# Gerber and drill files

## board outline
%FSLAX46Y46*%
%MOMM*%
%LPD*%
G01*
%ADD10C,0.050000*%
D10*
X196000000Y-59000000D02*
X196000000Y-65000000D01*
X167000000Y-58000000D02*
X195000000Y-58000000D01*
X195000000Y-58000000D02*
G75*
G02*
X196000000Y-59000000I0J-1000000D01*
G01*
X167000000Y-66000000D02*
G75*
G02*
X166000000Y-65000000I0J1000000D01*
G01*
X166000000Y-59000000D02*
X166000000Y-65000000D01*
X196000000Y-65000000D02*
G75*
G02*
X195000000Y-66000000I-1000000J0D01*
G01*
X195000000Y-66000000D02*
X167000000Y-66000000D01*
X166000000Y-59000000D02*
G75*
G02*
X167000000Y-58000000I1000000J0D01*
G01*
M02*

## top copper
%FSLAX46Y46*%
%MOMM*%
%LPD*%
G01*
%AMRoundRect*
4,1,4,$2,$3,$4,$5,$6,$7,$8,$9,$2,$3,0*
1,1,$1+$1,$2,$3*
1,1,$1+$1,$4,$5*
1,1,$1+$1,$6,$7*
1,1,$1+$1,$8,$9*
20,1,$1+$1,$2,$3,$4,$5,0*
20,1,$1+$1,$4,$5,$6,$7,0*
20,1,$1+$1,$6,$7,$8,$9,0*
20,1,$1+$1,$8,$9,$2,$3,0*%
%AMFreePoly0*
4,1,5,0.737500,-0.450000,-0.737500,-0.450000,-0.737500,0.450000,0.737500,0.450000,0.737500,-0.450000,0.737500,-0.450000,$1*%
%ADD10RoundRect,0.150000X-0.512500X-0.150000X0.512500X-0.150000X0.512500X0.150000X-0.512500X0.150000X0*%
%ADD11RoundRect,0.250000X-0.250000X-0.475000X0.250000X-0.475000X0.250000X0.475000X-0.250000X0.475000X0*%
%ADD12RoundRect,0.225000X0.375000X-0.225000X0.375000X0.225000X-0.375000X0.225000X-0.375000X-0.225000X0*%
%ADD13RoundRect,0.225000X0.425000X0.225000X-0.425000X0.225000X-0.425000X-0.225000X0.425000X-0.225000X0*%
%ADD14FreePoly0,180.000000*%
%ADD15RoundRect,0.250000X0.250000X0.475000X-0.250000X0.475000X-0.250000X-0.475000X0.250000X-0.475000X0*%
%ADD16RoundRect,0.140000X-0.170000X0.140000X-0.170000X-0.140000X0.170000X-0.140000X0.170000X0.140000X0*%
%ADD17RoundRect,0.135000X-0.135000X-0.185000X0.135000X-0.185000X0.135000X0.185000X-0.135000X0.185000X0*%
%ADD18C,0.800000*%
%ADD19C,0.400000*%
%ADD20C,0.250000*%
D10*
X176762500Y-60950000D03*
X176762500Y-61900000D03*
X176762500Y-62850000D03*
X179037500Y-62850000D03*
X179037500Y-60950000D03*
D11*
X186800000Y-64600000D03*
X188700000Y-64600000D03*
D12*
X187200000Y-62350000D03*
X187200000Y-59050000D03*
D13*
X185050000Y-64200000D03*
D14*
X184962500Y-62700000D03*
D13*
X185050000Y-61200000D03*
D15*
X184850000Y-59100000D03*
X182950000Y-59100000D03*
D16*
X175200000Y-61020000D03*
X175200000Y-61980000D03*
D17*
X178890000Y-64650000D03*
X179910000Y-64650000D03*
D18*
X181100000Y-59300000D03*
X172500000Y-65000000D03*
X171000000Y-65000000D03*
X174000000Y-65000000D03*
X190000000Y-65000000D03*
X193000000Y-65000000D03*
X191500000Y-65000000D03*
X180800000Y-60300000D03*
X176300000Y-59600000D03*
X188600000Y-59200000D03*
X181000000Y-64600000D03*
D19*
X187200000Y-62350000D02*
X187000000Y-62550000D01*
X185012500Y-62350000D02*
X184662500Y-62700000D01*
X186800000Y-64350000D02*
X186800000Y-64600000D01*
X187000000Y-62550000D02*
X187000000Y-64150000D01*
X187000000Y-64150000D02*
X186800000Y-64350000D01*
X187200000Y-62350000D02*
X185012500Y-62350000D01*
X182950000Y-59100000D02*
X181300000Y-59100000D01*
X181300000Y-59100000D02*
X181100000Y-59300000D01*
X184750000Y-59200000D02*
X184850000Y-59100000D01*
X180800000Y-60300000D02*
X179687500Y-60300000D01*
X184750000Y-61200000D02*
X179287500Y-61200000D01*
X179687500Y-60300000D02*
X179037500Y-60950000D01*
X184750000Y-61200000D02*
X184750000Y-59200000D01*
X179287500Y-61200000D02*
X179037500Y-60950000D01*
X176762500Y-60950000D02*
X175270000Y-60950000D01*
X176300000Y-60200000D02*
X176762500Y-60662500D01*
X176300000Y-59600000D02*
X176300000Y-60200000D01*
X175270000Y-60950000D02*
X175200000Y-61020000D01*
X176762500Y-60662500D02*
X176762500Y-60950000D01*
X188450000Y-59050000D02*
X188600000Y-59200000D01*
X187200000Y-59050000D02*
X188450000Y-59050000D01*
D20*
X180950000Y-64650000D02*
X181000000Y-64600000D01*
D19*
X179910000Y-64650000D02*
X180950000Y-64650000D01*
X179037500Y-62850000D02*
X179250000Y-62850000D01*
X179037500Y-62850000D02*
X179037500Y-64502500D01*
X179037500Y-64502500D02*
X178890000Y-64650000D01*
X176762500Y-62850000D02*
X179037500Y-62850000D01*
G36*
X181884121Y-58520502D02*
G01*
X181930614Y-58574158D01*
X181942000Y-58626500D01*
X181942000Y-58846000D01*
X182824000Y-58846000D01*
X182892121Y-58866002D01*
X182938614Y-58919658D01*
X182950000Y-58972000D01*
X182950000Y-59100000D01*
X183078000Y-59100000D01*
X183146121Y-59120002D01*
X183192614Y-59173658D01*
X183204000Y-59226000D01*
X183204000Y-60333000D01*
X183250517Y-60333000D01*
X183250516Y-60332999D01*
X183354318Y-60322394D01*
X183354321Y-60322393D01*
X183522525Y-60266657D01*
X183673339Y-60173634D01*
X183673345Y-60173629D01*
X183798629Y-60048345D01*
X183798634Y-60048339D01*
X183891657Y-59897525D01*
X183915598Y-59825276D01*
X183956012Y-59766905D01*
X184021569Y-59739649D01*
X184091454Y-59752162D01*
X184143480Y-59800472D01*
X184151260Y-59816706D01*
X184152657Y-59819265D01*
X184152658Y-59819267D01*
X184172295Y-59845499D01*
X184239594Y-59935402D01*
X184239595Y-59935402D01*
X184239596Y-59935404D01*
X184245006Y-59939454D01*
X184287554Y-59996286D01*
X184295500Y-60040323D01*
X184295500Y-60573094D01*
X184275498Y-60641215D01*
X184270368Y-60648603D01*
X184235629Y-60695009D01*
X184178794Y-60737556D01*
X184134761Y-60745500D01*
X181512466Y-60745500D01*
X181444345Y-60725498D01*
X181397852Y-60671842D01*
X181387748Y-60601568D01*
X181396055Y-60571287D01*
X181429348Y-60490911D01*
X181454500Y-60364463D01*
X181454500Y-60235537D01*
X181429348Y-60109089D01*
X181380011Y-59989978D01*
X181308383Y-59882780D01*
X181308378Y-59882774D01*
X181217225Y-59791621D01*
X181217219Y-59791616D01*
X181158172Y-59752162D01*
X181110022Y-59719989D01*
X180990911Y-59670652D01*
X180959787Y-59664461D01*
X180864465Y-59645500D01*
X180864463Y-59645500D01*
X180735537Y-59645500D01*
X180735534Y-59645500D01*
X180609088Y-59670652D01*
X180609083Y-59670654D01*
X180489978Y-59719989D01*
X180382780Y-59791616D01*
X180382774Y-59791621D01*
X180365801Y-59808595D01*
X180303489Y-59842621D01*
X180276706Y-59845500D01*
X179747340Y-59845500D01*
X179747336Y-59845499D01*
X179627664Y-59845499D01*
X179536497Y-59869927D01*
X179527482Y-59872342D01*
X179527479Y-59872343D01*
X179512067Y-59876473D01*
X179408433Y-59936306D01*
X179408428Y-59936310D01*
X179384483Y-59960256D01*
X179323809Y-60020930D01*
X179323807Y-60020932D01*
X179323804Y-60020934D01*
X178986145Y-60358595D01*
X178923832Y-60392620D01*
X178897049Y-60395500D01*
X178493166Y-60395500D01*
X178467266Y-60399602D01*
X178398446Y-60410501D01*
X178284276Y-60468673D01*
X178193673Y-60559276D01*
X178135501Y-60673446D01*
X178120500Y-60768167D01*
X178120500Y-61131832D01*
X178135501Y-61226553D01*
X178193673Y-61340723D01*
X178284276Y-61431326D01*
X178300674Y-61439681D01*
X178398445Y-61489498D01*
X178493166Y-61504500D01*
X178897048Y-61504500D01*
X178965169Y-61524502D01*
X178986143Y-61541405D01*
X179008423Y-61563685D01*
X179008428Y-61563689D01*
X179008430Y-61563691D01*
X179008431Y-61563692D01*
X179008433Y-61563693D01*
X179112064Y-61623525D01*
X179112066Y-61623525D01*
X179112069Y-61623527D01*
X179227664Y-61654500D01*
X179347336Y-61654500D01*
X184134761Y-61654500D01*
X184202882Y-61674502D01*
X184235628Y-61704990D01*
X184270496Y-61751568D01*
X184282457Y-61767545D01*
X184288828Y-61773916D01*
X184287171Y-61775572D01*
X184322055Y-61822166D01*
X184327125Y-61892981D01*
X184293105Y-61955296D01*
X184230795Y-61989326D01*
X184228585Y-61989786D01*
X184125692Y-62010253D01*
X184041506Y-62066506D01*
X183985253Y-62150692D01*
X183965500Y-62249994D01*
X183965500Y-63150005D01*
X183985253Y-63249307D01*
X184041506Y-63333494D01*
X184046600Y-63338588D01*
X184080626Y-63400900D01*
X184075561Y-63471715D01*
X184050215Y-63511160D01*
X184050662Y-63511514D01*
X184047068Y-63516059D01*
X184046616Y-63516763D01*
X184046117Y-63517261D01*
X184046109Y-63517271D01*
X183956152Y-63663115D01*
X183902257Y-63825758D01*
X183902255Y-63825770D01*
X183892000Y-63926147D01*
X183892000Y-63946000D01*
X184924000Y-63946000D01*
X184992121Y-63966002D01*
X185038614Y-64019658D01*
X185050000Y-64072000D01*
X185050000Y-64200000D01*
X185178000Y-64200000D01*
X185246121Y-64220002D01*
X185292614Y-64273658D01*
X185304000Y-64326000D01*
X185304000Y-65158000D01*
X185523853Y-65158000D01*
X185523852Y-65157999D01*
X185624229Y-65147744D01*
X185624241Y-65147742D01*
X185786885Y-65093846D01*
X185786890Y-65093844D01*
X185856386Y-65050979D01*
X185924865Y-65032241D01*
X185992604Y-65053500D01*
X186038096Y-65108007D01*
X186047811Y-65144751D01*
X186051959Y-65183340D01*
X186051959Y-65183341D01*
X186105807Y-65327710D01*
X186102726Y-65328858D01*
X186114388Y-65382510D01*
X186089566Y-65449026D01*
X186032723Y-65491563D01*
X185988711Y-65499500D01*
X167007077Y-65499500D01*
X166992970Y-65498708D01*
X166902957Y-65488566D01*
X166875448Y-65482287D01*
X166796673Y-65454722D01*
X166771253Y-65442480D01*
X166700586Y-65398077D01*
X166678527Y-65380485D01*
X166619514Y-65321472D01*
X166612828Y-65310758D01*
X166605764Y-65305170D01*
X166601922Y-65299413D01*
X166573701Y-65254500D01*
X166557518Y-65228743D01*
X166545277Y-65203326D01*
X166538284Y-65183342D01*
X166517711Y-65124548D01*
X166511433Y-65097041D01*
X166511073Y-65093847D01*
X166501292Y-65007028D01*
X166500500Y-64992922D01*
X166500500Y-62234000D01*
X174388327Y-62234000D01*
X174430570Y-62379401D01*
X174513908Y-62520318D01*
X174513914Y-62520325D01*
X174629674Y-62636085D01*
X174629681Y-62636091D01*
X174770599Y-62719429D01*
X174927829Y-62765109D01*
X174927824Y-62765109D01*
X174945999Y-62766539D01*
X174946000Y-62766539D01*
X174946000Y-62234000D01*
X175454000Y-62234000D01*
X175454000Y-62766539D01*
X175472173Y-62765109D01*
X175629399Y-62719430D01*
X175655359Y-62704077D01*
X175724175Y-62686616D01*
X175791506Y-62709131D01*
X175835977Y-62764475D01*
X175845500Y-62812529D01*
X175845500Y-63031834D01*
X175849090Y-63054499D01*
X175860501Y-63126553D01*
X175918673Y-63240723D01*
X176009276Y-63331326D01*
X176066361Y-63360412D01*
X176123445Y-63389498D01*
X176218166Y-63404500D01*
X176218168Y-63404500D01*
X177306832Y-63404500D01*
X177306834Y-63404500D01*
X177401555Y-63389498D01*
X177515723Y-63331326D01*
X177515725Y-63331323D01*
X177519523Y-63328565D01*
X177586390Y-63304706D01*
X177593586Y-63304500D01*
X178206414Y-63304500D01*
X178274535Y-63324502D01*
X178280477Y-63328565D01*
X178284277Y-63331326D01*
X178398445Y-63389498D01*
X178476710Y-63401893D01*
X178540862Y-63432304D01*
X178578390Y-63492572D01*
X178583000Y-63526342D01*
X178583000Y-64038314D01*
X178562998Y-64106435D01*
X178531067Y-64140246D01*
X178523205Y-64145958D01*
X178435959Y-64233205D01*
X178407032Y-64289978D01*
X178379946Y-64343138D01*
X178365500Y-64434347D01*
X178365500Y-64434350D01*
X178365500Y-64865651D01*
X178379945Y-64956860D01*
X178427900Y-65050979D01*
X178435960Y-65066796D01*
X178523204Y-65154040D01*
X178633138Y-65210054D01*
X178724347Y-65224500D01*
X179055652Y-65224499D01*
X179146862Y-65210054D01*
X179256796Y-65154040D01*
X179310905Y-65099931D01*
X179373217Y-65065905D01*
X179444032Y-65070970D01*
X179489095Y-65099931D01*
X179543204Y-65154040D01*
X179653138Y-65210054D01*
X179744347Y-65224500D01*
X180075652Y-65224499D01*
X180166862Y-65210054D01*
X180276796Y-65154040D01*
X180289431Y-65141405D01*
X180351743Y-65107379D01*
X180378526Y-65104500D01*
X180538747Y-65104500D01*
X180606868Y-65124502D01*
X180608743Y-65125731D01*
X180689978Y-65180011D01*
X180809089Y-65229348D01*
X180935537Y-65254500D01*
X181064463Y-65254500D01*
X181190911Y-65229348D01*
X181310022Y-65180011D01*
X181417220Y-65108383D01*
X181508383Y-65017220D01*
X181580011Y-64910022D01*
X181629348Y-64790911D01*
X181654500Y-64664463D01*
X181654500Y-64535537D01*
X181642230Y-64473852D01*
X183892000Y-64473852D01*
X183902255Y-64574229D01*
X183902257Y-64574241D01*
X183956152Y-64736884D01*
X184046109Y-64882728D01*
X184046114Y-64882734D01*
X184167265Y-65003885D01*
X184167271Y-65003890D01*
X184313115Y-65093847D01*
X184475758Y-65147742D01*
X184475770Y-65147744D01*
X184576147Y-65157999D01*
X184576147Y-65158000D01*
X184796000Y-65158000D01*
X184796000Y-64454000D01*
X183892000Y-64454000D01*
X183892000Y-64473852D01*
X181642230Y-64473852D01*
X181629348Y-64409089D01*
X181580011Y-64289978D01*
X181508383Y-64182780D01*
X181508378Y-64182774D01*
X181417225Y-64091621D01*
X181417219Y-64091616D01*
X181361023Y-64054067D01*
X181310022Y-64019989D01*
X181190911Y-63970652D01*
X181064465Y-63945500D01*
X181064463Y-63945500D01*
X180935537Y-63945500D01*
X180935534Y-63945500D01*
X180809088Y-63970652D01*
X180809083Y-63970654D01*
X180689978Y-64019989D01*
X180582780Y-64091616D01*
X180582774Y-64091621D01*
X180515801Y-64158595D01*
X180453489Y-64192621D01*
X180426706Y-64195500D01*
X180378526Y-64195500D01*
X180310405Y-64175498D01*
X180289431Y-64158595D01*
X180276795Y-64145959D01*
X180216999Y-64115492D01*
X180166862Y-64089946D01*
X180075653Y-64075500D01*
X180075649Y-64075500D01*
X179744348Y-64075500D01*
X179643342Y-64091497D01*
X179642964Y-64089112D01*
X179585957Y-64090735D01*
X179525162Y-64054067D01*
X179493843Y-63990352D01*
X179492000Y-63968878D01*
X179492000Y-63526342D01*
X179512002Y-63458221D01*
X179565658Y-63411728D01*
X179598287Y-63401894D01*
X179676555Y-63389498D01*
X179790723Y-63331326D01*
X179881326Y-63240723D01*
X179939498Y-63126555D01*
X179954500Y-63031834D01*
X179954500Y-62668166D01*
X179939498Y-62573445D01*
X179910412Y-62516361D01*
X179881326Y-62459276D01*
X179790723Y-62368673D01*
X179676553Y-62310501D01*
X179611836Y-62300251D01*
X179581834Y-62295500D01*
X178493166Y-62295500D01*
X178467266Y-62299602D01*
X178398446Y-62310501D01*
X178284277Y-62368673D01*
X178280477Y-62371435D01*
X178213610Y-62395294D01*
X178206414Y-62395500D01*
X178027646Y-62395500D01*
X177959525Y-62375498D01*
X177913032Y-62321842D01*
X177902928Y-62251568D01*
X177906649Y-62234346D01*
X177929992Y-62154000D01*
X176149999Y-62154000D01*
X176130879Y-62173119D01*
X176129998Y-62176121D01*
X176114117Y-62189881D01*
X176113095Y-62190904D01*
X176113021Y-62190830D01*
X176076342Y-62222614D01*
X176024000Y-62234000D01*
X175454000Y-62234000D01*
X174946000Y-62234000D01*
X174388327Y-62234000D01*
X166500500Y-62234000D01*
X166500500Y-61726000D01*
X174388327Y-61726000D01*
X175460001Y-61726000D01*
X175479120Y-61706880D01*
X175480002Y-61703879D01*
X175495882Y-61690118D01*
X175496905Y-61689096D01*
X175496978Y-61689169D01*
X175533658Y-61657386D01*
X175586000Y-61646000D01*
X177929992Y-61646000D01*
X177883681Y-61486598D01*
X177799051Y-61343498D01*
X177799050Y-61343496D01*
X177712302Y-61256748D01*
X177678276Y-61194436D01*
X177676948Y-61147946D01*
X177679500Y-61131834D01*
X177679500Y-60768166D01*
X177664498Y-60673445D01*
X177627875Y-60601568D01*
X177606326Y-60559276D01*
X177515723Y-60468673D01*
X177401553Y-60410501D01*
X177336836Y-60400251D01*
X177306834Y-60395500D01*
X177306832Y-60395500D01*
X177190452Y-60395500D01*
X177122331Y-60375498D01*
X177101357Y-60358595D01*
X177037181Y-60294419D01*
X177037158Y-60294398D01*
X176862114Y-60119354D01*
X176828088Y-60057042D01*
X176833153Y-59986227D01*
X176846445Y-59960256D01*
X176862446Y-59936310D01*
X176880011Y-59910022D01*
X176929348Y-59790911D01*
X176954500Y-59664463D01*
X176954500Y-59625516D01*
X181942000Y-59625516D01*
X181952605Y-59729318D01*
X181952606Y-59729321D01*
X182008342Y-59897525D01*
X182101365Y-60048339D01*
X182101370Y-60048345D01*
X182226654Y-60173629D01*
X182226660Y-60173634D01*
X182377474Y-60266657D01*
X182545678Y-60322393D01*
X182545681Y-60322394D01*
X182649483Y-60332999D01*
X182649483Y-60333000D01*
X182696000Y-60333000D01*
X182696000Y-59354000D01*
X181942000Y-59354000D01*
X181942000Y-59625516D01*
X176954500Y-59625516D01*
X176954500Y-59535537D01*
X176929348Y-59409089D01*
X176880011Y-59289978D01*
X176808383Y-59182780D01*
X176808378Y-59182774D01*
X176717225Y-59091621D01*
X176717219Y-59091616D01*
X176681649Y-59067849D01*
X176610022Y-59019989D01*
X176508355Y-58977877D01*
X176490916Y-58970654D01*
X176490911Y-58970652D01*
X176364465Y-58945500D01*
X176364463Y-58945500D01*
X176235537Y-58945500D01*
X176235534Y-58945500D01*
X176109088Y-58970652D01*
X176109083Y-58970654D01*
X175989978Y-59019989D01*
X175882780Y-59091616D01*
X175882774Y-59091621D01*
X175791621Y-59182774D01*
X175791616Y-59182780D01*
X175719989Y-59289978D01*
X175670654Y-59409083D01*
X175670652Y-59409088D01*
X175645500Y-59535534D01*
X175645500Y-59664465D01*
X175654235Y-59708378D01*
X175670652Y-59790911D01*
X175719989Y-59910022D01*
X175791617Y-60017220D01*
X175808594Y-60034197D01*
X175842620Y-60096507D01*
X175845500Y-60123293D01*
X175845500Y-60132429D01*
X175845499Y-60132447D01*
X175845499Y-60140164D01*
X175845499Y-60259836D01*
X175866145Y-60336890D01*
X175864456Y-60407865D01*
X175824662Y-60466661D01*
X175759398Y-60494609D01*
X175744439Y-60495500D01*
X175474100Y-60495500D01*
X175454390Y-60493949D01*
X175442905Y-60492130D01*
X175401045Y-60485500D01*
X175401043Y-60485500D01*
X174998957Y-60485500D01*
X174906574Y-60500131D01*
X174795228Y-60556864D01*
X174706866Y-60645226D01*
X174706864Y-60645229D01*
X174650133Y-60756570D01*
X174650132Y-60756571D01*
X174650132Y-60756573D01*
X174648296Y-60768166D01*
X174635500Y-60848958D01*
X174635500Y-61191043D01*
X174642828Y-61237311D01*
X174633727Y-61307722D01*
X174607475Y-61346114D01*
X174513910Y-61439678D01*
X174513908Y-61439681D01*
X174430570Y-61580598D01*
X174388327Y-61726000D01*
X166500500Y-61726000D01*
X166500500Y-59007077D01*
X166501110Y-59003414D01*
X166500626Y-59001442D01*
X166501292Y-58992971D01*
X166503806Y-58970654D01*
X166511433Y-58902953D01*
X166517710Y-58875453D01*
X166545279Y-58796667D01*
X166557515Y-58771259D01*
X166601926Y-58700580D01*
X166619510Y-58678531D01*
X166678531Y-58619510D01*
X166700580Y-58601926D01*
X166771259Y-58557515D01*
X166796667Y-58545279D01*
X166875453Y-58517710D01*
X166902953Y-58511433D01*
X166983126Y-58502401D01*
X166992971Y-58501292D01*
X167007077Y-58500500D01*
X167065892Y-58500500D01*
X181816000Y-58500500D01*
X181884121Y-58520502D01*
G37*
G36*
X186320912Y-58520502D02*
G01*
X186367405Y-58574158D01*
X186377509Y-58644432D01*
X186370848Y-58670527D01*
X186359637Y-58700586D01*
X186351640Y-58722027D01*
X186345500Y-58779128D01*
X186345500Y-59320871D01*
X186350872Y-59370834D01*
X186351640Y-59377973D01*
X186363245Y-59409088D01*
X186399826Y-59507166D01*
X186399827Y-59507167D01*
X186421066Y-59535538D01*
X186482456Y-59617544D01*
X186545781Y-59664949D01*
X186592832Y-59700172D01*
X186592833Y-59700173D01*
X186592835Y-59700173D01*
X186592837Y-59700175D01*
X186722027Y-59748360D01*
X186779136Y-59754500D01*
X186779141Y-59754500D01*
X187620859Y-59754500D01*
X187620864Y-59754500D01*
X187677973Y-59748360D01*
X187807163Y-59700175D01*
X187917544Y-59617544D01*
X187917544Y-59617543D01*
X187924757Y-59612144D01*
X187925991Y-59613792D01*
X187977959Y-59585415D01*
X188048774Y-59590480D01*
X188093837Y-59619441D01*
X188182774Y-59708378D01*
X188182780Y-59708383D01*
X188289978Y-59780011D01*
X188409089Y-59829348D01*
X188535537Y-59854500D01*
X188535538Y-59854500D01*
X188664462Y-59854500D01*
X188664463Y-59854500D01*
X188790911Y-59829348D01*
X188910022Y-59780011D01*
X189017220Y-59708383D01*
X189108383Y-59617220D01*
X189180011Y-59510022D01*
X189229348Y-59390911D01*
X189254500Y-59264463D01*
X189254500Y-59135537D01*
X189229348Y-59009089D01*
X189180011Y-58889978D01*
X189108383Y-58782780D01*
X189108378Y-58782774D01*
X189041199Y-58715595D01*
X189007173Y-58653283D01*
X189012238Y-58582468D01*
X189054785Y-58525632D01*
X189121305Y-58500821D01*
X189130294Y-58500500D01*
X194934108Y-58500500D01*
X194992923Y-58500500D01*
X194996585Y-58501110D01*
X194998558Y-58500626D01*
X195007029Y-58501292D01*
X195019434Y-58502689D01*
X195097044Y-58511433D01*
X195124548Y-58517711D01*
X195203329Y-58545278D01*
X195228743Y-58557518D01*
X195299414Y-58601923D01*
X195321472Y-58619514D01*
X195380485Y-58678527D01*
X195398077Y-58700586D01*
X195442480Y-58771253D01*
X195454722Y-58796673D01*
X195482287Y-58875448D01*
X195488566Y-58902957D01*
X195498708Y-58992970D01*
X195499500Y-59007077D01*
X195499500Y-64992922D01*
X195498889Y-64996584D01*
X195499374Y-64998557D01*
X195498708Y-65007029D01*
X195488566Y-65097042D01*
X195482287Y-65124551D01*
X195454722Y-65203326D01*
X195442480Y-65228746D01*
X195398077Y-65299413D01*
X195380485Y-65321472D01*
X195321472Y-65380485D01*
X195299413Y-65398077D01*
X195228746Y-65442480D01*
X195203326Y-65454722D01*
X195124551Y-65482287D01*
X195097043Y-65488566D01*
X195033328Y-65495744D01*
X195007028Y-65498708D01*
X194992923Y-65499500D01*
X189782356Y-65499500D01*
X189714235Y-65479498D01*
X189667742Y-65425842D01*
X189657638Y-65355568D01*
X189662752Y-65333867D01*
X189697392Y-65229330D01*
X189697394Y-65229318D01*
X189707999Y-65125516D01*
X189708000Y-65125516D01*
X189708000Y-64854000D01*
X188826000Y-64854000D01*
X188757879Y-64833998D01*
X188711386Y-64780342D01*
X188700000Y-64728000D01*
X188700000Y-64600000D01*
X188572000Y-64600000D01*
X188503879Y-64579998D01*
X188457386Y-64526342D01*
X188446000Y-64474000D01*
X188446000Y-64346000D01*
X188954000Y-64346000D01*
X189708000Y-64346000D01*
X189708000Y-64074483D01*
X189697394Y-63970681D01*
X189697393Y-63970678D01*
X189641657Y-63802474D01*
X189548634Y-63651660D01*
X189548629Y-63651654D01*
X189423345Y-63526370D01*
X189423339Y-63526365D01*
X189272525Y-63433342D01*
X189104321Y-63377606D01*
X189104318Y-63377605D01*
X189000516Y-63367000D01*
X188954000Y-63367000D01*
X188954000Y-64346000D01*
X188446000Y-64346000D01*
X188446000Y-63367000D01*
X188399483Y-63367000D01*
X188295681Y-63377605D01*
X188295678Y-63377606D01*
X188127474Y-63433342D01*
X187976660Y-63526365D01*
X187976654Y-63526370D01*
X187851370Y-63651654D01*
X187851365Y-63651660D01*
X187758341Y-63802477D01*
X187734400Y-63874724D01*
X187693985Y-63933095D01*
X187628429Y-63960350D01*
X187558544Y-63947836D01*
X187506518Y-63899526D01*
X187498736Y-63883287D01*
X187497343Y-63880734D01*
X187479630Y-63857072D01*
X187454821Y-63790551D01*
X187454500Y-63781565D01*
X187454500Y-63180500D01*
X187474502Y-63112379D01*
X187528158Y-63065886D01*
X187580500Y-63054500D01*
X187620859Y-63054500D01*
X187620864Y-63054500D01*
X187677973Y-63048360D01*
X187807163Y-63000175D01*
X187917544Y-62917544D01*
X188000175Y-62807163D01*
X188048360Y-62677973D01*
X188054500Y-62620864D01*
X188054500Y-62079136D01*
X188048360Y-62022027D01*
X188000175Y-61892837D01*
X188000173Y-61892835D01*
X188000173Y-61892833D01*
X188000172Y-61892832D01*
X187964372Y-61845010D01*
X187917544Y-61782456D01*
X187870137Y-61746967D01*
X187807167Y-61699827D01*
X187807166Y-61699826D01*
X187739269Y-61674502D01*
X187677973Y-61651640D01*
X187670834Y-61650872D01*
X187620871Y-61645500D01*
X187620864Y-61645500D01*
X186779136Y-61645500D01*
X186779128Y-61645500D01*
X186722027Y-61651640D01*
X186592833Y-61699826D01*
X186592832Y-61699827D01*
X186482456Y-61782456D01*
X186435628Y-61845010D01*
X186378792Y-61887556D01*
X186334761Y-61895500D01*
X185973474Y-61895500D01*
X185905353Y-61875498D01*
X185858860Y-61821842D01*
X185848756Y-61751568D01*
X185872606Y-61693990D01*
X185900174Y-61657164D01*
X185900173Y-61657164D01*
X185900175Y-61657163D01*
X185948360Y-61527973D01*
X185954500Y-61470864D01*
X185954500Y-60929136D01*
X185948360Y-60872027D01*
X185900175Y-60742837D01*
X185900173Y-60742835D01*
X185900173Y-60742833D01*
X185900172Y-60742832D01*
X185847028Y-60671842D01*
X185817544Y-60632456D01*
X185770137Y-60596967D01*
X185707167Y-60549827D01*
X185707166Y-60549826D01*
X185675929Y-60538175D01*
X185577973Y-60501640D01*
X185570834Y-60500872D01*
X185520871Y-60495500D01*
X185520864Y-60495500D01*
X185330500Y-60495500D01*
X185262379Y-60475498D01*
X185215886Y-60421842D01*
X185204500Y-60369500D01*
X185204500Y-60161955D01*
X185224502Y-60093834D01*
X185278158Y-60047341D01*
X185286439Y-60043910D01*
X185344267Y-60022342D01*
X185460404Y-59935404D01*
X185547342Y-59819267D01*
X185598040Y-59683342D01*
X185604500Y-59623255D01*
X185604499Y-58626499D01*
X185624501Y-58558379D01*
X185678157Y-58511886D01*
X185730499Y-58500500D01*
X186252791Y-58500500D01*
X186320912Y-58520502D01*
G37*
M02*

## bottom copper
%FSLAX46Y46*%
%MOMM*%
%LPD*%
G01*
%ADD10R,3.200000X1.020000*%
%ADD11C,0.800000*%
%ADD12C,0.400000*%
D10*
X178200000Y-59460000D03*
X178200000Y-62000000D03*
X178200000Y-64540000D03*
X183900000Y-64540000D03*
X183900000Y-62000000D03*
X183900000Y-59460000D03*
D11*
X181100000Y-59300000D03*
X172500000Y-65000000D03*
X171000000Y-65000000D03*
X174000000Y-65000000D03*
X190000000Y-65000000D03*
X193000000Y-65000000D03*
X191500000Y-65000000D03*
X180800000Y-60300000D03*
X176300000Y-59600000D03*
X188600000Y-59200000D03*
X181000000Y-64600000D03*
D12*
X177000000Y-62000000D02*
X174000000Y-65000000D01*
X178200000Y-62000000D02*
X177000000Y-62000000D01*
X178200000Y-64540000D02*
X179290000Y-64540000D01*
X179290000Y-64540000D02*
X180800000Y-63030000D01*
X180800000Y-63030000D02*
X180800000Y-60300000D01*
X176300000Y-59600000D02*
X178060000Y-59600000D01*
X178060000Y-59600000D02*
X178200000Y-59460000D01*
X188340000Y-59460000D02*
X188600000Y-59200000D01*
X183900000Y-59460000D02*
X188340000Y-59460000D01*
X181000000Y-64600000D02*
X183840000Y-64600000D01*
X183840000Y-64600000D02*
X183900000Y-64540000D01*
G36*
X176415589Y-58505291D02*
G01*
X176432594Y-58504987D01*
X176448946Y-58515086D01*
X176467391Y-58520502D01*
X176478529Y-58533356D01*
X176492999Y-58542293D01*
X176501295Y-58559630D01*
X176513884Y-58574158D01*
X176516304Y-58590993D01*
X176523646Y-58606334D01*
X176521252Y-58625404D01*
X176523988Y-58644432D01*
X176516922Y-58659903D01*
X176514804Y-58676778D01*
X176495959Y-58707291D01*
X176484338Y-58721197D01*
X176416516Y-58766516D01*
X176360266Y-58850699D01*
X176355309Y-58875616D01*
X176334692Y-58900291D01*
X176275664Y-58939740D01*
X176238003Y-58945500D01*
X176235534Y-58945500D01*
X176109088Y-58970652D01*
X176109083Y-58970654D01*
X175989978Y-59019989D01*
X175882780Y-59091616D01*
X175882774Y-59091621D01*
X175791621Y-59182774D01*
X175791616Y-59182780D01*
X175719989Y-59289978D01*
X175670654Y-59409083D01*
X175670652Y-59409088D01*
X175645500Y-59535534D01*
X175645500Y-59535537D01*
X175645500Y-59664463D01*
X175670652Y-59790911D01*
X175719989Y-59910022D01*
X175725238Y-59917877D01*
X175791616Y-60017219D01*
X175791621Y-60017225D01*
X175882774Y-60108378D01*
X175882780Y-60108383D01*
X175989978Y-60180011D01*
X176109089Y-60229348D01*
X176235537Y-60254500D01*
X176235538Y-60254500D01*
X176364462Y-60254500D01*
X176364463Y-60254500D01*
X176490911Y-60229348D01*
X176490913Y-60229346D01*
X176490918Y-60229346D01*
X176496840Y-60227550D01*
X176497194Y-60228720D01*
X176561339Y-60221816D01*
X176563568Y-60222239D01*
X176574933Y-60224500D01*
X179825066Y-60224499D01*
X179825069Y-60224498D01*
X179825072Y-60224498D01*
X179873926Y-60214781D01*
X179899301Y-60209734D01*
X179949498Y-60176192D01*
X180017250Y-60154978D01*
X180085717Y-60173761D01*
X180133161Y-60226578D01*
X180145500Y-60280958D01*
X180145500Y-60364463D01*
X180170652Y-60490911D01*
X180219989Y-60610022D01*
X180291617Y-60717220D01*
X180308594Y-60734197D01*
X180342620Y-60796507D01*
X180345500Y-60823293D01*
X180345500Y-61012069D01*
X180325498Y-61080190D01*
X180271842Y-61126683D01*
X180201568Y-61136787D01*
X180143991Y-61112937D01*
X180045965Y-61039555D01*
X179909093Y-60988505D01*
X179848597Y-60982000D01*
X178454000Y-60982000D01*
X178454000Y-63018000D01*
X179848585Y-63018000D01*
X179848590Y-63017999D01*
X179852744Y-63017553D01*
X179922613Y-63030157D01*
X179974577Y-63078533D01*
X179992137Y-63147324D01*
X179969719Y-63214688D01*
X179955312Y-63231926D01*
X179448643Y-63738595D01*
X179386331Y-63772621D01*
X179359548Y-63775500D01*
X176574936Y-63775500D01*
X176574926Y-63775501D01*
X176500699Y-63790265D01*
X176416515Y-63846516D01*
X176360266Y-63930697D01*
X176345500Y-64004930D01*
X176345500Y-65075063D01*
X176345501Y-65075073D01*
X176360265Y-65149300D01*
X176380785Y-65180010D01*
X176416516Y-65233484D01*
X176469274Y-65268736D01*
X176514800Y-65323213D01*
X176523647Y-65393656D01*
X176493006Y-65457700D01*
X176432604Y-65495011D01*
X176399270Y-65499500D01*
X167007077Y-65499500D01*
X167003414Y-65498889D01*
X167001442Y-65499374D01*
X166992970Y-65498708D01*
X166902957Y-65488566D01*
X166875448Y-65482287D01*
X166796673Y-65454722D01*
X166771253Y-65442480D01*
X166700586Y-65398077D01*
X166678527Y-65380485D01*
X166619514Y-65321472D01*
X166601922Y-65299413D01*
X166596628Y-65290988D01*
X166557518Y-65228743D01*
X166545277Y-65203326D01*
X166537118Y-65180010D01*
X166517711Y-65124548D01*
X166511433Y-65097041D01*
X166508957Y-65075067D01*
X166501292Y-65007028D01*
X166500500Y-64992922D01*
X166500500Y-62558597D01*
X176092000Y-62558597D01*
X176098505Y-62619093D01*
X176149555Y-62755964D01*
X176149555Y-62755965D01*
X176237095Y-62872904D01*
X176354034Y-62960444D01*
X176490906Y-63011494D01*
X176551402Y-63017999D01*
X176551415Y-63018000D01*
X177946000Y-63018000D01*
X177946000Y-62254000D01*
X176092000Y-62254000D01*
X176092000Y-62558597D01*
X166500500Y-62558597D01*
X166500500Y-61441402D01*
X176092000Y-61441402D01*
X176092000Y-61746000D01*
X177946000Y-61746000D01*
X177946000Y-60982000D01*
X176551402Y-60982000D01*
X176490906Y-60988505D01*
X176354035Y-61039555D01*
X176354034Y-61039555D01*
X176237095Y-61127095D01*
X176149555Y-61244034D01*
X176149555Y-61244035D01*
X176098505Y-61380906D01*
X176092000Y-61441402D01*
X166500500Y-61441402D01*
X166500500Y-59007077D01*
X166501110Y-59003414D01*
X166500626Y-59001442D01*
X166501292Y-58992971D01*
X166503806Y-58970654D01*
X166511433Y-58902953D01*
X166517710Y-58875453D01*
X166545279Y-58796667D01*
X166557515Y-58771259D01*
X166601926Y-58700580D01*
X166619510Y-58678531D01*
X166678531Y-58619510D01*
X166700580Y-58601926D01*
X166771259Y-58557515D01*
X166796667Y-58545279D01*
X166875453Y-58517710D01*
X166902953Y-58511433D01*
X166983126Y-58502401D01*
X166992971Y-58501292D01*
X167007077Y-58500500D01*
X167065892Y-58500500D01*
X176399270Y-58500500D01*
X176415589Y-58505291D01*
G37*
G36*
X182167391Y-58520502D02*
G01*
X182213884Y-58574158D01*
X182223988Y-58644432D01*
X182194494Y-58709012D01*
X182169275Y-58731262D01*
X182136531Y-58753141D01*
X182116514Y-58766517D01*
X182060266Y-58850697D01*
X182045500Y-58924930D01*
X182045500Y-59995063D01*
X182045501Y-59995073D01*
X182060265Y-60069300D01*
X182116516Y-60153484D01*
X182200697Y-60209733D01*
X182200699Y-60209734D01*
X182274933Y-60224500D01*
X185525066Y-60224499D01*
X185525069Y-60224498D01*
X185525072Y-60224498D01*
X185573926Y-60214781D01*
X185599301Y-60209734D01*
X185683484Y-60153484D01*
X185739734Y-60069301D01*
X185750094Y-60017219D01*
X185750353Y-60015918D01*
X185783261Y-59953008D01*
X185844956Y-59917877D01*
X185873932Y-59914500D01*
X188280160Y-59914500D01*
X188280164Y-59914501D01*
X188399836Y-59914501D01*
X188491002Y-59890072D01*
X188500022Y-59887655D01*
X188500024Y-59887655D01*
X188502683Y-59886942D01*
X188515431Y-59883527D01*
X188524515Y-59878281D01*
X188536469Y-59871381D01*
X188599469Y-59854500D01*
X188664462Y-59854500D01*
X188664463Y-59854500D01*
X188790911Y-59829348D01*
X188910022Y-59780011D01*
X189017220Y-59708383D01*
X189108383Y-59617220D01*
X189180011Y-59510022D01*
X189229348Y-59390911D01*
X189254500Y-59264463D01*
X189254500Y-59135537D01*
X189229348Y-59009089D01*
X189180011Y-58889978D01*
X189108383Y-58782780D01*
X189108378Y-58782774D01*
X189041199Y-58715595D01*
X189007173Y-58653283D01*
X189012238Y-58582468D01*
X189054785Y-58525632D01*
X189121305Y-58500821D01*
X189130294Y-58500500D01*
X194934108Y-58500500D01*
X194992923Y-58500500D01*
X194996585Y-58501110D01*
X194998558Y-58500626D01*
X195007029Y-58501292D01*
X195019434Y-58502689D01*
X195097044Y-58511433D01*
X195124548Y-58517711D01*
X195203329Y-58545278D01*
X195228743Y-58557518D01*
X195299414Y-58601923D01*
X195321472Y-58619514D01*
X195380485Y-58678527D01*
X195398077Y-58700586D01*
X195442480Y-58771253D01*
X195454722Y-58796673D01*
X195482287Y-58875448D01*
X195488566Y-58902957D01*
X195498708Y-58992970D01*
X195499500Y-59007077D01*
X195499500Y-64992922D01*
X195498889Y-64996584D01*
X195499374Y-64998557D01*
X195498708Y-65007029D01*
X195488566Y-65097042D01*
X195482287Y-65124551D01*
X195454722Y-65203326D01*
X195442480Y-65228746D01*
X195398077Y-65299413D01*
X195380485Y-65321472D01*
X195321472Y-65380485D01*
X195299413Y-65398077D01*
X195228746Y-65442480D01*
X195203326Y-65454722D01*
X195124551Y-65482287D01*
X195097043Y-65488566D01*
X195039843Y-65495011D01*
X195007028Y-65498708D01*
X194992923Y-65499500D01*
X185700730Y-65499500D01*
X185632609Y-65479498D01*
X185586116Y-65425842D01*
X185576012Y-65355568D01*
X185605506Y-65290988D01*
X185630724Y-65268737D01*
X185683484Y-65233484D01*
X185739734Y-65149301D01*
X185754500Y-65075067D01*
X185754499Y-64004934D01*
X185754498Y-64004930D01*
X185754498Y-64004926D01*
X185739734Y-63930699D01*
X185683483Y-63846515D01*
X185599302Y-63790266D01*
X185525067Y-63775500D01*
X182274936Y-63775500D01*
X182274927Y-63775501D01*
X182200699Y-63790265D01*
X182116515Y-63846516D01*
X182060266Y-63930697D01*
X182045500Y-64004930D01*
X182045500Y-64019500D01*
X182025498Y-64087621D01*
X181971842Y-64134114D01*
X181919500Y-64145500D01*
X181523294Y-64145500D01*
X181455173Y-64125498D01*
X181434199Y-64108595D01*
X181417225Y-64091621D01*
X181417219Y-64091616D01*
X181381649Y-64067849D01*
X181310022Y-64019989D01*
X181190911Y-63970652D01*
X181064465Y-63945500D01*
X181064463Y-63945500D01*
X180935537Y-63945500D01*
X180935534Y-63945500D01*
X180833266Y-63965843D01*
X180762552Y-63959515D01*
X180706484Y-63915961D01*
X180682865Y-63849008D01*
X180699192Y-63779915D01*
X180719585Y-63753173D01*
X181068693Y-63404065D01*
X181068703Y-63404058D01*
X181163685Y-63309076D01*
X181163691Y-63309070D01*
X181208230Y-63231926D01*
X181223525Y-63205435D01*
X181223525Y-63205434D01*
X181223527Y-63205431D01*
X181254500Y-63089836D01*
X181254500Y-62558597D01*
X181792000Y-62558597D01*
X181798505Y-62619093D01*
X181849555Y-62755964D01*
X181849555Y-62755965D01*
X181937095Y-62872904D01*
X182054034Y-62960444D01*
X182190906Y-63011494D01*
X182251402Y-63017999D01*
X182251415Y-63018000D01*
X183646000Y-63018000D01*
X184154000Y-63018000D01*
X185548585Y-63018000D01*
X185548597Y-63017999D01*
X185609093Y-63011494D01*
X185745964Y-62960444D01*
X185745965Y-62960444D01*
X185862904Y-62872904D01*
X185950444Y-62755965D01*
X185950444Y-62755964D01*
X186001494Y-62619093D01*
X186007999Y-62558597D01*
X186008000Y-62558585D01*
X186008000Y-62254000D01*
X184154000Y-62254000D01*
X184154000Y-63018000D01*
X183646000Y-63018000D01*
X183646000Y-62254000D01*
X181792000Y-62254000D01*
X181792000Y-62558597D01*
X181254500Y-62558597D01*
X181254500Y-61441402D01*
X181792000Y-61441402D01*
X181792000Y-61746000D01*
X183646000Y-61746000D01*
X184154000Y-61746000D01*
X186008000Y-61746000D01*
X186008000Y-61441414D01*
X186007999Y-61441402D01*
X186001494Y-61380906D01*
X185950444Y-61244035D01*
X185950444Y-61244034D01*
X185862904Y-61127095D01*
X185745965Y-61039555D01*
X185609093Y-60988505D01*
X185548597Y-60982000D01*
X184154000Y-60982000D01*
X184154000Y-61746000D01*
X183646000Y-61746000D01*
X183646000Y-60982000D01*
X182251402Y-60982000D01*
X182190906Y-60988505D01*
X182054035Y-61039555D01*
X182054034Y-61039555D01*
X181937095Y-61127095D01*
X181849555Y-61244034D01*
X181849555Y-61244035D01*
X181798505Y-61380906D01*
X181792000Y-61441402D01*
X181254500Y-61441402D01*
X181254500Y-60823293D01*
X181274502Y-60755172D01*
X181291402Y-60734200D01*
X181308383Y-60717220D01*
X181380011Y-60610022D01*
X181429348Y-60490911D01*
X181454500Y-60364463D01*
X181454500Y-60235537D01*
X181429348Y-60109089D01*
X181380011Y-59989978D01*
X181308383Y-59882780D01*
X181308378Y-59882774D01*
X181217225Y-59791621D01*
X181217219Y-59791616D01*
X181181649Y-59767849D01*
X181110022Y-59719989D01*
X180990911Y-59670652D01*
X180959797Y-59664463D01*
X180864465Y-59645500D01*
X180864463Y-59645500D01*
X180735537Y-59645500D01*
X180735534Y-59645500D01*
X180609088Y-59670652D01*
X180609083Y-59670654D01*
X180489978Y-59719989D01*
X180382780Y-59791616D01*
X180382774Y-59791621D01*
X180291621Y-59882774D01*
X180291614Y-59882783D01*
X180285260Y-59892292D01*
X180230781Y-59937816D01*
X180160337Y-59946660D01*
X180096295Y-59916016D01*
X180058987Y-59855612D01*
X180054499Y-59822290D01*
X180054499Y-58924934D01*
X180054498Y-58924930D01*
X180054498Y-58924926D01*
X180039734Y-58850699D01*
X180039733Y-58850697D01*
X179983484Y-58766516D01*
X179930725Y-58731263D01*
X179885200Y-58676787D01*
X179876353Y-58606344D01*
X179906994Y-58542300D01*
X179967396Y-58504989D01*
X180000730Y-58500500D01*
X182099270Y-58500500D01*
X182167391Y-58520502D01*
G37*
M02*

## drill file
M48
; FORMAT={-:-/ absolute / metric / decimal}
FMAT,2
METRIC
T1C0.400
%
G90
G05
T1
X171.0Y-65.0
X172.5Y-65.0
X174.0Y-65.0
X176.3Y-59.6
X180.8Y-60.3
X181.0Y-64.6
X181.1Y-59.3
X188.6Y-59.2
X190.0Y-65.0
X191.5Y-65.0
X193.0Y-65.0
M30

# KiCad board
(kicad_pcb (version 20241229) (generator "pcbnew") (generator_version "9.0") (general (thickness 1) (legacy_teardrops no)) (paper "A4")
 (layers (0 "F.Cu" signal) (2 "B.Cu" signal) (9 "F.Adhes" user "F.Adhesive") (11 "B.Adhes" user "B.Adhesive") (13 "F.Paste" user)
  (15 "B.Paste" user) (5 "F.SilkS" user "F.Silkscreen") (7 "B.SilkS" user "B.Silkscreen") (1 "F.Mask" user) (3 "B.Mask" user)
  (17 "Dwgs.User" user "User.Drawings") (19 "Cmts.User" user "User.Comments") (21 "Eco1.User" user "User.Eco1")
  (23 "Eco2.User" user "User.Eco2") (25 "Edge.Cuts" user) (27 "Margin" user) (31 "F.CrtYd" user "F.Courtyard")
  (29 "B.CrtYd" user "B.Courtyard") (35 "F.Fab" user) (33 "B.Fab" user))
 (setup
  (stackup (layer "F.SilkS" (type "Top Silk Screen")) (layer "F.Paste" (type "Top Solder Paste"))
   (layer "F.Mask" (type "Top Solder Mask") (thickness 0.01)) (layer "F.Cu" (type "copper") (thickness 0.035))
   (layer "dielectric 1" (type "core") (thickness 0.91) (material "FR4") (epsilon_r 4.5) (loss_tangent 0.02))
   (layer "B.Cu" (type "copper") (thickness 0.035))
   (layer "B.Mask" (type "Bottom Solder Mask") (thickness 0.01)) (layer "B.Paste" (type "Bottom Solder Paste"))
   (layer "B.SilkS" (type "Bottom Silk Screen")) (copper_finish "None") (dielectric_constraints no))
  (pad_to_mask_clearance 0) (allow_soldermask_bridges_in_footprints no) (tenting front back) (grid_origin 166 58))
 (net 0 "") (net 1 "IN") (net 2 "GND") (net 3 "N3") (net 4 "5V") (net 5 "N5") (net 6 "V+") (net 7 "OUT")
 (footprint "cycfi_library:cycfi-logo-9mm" (layer "F.Cu") (at 171.25 59.4)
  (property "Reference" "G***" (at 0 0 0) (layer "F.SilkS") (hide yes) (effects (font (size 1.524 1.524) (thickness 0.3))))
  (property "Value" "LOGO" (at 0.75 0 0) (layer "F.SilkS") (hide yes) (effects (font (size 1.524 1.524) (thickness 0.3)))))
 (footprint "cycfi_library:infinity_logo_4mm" (layer "F.Cu") (at 192.3 60.2)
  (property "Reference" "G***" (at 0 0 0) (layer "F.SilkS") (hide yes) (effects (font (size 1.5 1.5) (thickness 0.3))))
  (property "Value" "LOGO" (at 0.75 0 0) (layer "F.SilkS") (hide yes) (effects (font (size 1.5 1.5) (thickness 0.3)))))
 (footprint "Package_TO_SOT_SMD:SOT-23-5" (layer "F.Cu") (at 177.9 61.9)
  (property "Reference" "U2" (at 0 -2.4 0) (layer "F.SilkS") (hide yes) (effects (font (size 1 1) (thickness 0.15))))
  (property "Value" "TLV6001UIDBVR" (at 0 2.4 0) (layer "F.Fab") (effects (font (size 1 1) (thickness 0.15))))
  (pad "1" smd roundrect (at -1.1375 -0.95) (size 1.325 0.6) (layers "F.Cu" "F.Mask" "F.Paste") (roundrect_rratio 0.25) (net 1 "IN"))
  (pad "2" smd roundrect (at -1.1375 0) (size 1.325 0.6) (layers "F.Cu" "F.Mask" "F.Paste") (roundrect_rratio 0.25) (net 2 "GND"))
  (pad "3" smd roundrect (at -1.1375 0.95) (size 1.325 0.6) (layers "F.Cu" "F.Mask" "F.Paste") (roundrect_rratio 0.25) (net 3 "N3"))
  (pad "4" smd roundrect (at 1.1375 0.95) (size 1.325 0.6) (layers "F.Cu" "F.Mask" "F.Paste") (roundrect_rratio 0.25) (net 3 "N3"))
  (pad "5" smd roundrect (at 1.1375 -0.95) (size 1.325 0.6) (layers "F.Cu" "F.Mask" "F.Paste") (roundrect_rratio 0.25) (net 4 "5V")))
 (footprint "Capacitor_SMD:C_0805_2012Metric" (layer "F.Cu") (at 187.75 64.6)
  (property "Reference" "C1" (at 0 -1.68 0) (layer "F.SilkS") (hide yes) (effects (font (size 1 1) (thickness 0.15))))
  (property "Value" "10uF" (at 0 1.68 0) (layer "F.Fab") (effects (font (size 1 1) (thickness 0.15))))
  (pad "1" smd roundrect (at -0.95 0) (size 1 1.45) (layers "F.Cu" "F.Mask" "F.Paste") (roundrect_rratio 0.25) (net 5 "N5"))
  (pad "2" smd roundrect (at 0.95 0) (size 1 1.45) (layers "F.Cu" "F.Mask" "F.Paste") (roundrect_rratio 0.25) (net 2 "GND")))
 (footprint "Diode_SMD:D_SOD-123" (layer "F.Cu") (at 187.2 60.7 90)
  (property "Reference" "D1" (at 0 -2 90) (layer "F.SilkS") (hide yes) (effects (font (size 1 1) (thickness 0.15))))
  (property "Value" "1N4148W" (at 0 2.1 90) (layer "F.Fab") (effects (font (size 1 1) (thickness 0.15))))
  (pad "1" smd roundrect (at -1.65 0 90) (size 0.9 1.2) (layers "F.Cu" "F.Mask" "F.Paste") (roundrect_rratio 0.25) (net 5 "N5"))
  (pad "2" smd roundrect (at 1.65 0 90) (size 0.9 1.2) (layers "F.Cu" "F.Mask" "F.Paste") (roundrect_rratio 0.25) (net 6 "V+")))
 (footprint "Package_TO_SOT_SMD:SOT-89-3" (layer "F.Cu") (at 183.1 62.7 180)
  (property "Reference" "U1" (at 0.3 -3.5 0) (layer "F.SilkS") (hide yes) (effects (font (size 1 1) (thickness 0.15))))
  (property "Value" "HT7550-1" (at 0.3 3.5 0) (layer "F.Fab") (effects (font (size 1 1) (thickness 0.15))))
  (pad "1" smd roundrect (at -1.95 -1.5 180) (size 1.3 0.9) (layers "F.Cu" "F.Mask" "F.Paste") (roundrect_rratio 0.25) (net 2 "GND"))
  (pad "2" smd custom (at -1.8625 0 180) (size 1.475 0.9) (layers "F.Cu" "F.Mask" "F.Paste") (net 5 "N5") (zone_connect 2)
   (thermal_bridge_angle 45) (options (clearance outline) (anchor rect)) (primitives))
  (pad "3" smd roundrect (at -1.95 1.5 180) (size 1.3 0.9) (layers "F.Cu" "F.Mask" "F.Paste") (roundrect_rratio 0.25) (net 4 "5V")))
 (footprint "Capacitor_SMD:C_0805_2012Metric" (layer "F.Cu") (at 183.9 59.1 180)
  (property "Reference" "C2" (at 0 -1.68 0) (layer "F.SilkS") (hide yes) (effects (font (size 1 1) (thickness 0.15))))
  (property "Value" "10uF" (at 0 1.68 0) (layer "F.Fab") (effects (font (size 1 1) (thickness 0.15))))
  (pad "1" smd roundrect (at -0.95 0 180) (size 1 1.45) (layers "F.Cu" "F.Mask" "F.Paste") (roundrect_rratio 0.25) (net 4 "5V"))
  (pad "2" smd roundrect (at 0.95 0 180) (size 1 1.45) (layers "F.Cu" "F.Mask" "F.Paste") (roundrect_rratio 0.25) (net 2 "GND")))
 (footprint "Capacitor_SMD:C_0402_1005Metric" (layer "F.Cu") (at 175.2 61.5 -90)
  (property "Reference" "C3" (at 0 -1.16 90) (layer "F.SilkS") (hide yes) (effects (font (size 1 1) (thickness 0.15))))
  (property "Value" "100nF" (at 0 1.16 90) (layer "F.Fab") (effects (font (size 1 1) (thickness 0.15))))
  (pad "1" smd roundrect (at -0.48 0 270) (size 0.56 0.62) (layers "F.Cu" "F.Mask" "F.Paste") (roundrect_rratio 0.25) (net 1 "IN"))
  (pad "2" smd roundrect (at 0.48 0 270) (size 0.56 0.62) (layers "F.Cu" "F.Mask" "F.Paste") (roundrect_rratio 0.25) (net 2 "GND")))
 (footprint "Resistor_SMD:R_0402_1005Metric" (layer "F.Cu") (at 179.4 64.65)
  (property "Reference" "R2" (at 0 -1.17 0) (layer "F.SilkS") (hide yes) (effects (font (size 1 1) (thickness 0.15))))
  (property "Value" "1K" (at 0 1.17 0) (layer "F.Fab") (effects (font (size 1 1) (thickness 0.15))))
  (pad "1" smd roundrect (at -0.51 0) (size 0.54 0.64) (layers "F.Cu" "F.Mask" "F.Paste") (roundrect_rratio 0.25) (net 3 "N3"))
  (pad "2" smd roundrect (at 0.51 0) (size 0.54 0.64) (layers "F.Cu" "F.Mask" "F.Paste") (roundrect_rratio 0.25) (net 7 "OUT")))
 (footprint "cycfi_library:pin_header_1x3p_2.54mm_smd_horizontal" (layer "B.Cu") (at 178.2 62 180)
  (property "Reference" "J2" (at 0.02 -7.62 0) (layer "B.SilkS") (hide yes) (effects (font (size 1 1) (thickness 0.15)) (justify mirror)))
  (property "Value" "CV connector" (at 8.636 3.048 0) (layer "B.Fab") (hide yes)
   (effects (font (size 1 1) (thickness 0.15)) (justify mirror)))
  (pad "1" smd rect (at 0 2.54 180) (size 3.2 1.02) (layers "B.Cu" "B.Mask" "B.Paste") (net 1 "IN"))
  (pad "2" smd rect (at 0 0 180) (size 3.2 1.02) (layers "B.Cu" "B.Mask" "B.Paste") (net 2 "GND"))
  (pad "3" smd rect (at 0 -2.54 180) (size 3.2 1.02) (layers "B.Cu" "B.Mask" "B.Paste") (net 4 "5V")))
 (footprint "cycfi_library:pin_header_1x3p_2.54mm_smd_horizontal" (layer "B.Cu") (at 183.9 62)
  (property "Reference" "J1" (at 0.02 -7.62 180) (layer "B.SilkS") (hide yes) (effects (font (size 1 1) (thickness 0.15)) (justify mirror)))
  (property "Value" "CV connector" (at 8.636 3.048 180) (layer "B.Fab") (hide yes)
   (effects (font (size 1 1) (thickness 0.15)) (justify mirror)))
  (pad "1" smd rect (at 0 2.54) (size 3.2 1.02) (layers "B.Cu" "B.Mask" "B.Paste") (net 7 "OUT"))
  (pad "2" smd rect (at 0 0) (size 3.2 1.02) (layers "B.Cu" "B.Mask" "B.Paste") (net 2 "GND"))
  (pad "3" smd rect (at 0 -2.54) (size 3.2 1.02) (layers "B.Cu" "B.Mask" "B.Paste") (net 6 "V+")))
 (gr_line (start 196 59) (end 196 65) (stroke (width 0.05) (type solid)) (layer "Edge.Cuts"))
 (gr_line (start 167 58) (end 195 58) (stroke (width 0.05) (type solid)) (layer "Edge.Cuts"))
 (gr_arc (start 195 58) (mid 195.707107 58.292893) (end 196 59) (stroke (width 0.05) (type solid)) (layer "Edge.Cuts"))
 (gr_arc (start 167 66) (mid 166.292893 65.707107) (end 166 65) (stroke (width 0.05) (type solid)) (layer "Edge.Cuts"))
 (gr_line (start 166 59) (end 166 65) (stroke (width 0.05) (type solid)) (layer "Edge.Cuts"))
 (gr_arc (start 196 65) (mid 195.707107 65.707107) (end 195 66) (stroke (width 0.05) (type solid)) (layer "Edge.Cuts"))
 (gr_line (start 195 66) (end 167 66) (stroke (width 0.05) (type solid)) (layer "Edge.Cuts"))
 (gr_arc (start 166 59) (mid 166.292893 58.292893) (end 167 58) (stroke (width 0.05) (type solid)) (layer "Edge.Cuts"))
 (segment (start 187.2 62.35) (end 187 62.55) (width 0.4) (layer "F.Cu") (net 5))
 (segment (start 185.0125 62.35) (end 184.6625 62.7) (width 0.4) (layer "F.Cu") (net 5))
 (segment (start 186.8 64.35) (end 186.8 64.6) (width 0.4) (layer "F.Cu") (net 5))
 (segment (start 187 62.55) (end 187 64.15) (width 0.4) (layer "F.Cu") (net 5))
 (segment (start 187 64.15) (end 186.8 64.35) (width 0.4) (layer "F.Cu") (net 5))
 (segment (start 187.2 62.35) (end 185.0125 62.35) (width 0.4) (layer "F.Cu") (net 5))
 (segment (start 182.95 59.1) (end 181.3 59.1) (width 0.4) (layer "F.Cu") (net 2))
 (segment (start 181.3 59.1) (end 181.1 59.3) (width 0.4) (layer "F.Cu") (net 2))
 (via (at 181.1 59.3) (size 0.8) (drill 0.4) (layers "F.Cu" "B.Cu") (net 2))
 (via (at 172.5 65) (size 0.8) (drill 0.4) (layers "F.Cu" "B.Cu") (free yes) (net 2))
 (via (at 171 65) (size 0.8) (drill 0.4) (layers "F.Cu" "B.Cu") (free yes) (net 2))
 (via (at 174 65) (size 0.8) (drill 0.4) (layers "F.Cu" "B.Cu") (free yes) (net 2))
 (via (at 190 65) (size 0.8) (drill 0.4) (layers "F.Cu" "B.Cu") (free yes) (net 2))
 (via (at 193 65) (size 0.8) (drill 0.4) (layers "F.Cu" "B.Cu") (free yes) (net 2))
 (via (at 191.5 65) (size 0.8) (drill 0.4) (layers "F.Cu" "B.Cu") (free yes) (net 2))
 (segment (start 177 62) (end 174 65) (width 0.4) (layer "B.Cu") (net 2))
 (segment (start 178.2 62) (end 177 62) (width 0.4) (layer "B.Cu") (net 2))
 (segment (start 184.75 59.2) (end 184.85 59.1) (width 0.4) (layer "F.Cu") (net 4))
 (segment (start 180.8 60.3) (end 179.6875 60.3) (width 0.4) (layer "F.Cu") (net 4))
 (segment (start 184.75 61.2) (end 179.2875 61.2) (width 0.4) (layer "F.Cu") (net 4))
 (segment (start 179.6875 60.3) (end 179.0375 60.95) (width 0.4) (layer "F.Cu") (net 4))
 (segment (start 184.75 61.2) (end 184.75 59.2) (width 0.4) (layer "F.Cu") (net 4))
 (segment (start 179.2875 61.2) (end 179.0375 60.95) (width 0.4) (layer "F.Cu") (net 4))
 (via (at 180.8 60.3) (size 0.8) (drill 0.4) (layers "F.Cu" "B.Cu") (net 4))
 (segment (start 178.2 64.54) (end 179.29 64.54) (width 0.4) (layer "B.Cu") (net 4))
 (segment (start 179.29 64.54) (end 180.8 63.03) (width 0.4) (layer "B.Cu") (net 4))
 (segment (start 180.8 63.03) (end 180.8 60.3) (width 0.4) (layer "B.Cu") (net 4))
 (segment (start 176.7625 60.95) (end 175.27 60.95) (width 0.4) (layer "F.Cu") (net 1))
 (segment (start 176.3 60.2) (end 176.7625 60.6625) (width 0.4) (layer "F.Cu") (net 1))
 (segment (start 176.3 59.6) (end 176.3 60.2) (width 0.4) (layer "F.Cu") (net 1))
 (segment (start 175.27 60.95) (end 175.2 61.02) (width 0.4) (layer "F.Cu") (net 1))
 (segment (start 176.7625 60.6625) (end 176.7625 60.95) (width 0.4) (layer "F.Cu") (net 1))
 (via (at 176.3 59.6) (size 0.8) (drill 0.4) (layers "F.Cu" "B.Cu") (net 1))
 (segment (start 176.3 59.6) (end 178.06 59.6) (width 0.4) (layer "B.Cu") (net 1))
 (segment (start 178.06 59.6) (end 178.2 59.46) (width 0.4) (layer "B.Cu") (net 1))
 (segment (start 188.45 59.05) (end 188.6 59.2) (width 0.4) (layer "F.Cu") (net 6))
 (segment (start 187.2 59.05) (end 188.45 59.05) (width 0.4) (layer "F.Cu") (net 6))
 (via (at 188.6 59.2) (size 0.8) (drill 0.4) (layers "F.Cu" "B.Cu") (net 6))
 (segment (start 188.34 59.46) (end 188.6 59.2) (width 0.4) (layer "B.Cu") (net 6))
 (segment (start 183.9 59.46) (end 188.34 59.46) (width 0.4) (layer "B.Cu") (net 6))
 (segment (start 180.95 64.65) (end 181 64.6) (width 0.25) (layer "F.Cu") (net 7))
 (segment (start 179.91 64.65) (end 180.95 64.65) (width 0.4) (layer "F.Cu") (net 7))
 (via (at 181 64.6) (size 0.8) (drill 0.4) (layers "F.Cu" "B.Cu") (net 7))
 (segment (start 181 64.6) (end 183.84 64.6) (width 0.4) (layer "B.Cu") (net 7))
 (segment (start 183.84 64.6) (end 183.9 64.54) (width 0.4) (layer "B.Cu") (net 7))
 (segment (start 179.0375 62.85) (end 179.25 62.85) (width 0.4) (layer "F.Cu") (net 3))
 (segment (start 179.0375 62.85) (end 179.0375 64.5025) (width 0.4) (layer "F.Cu") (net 3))
 (segment (start 179.0375 64.5025) (end 178.89 64.65) (width 0.4) (layer "F.Cu") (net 3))
 (segment (start 176.7625 62.85) (end 179.0375 62.85) (width 0.4) (layer "F.Cu") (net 3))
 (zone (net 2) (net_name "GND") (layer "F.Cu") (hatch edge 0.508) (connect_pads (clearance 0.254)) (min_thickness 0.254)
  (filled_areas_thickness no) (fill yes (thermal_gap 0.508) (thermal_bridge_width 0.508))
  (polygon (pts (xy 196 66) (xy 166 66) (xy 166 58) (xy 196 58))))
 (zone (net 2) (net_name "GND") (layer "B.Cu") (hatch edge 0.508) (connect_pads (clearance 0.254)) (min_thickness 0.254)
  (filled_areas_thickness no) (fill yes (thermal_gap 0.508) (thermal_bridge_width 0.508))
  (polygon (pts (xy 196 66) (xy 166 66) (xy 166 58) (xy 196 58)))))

